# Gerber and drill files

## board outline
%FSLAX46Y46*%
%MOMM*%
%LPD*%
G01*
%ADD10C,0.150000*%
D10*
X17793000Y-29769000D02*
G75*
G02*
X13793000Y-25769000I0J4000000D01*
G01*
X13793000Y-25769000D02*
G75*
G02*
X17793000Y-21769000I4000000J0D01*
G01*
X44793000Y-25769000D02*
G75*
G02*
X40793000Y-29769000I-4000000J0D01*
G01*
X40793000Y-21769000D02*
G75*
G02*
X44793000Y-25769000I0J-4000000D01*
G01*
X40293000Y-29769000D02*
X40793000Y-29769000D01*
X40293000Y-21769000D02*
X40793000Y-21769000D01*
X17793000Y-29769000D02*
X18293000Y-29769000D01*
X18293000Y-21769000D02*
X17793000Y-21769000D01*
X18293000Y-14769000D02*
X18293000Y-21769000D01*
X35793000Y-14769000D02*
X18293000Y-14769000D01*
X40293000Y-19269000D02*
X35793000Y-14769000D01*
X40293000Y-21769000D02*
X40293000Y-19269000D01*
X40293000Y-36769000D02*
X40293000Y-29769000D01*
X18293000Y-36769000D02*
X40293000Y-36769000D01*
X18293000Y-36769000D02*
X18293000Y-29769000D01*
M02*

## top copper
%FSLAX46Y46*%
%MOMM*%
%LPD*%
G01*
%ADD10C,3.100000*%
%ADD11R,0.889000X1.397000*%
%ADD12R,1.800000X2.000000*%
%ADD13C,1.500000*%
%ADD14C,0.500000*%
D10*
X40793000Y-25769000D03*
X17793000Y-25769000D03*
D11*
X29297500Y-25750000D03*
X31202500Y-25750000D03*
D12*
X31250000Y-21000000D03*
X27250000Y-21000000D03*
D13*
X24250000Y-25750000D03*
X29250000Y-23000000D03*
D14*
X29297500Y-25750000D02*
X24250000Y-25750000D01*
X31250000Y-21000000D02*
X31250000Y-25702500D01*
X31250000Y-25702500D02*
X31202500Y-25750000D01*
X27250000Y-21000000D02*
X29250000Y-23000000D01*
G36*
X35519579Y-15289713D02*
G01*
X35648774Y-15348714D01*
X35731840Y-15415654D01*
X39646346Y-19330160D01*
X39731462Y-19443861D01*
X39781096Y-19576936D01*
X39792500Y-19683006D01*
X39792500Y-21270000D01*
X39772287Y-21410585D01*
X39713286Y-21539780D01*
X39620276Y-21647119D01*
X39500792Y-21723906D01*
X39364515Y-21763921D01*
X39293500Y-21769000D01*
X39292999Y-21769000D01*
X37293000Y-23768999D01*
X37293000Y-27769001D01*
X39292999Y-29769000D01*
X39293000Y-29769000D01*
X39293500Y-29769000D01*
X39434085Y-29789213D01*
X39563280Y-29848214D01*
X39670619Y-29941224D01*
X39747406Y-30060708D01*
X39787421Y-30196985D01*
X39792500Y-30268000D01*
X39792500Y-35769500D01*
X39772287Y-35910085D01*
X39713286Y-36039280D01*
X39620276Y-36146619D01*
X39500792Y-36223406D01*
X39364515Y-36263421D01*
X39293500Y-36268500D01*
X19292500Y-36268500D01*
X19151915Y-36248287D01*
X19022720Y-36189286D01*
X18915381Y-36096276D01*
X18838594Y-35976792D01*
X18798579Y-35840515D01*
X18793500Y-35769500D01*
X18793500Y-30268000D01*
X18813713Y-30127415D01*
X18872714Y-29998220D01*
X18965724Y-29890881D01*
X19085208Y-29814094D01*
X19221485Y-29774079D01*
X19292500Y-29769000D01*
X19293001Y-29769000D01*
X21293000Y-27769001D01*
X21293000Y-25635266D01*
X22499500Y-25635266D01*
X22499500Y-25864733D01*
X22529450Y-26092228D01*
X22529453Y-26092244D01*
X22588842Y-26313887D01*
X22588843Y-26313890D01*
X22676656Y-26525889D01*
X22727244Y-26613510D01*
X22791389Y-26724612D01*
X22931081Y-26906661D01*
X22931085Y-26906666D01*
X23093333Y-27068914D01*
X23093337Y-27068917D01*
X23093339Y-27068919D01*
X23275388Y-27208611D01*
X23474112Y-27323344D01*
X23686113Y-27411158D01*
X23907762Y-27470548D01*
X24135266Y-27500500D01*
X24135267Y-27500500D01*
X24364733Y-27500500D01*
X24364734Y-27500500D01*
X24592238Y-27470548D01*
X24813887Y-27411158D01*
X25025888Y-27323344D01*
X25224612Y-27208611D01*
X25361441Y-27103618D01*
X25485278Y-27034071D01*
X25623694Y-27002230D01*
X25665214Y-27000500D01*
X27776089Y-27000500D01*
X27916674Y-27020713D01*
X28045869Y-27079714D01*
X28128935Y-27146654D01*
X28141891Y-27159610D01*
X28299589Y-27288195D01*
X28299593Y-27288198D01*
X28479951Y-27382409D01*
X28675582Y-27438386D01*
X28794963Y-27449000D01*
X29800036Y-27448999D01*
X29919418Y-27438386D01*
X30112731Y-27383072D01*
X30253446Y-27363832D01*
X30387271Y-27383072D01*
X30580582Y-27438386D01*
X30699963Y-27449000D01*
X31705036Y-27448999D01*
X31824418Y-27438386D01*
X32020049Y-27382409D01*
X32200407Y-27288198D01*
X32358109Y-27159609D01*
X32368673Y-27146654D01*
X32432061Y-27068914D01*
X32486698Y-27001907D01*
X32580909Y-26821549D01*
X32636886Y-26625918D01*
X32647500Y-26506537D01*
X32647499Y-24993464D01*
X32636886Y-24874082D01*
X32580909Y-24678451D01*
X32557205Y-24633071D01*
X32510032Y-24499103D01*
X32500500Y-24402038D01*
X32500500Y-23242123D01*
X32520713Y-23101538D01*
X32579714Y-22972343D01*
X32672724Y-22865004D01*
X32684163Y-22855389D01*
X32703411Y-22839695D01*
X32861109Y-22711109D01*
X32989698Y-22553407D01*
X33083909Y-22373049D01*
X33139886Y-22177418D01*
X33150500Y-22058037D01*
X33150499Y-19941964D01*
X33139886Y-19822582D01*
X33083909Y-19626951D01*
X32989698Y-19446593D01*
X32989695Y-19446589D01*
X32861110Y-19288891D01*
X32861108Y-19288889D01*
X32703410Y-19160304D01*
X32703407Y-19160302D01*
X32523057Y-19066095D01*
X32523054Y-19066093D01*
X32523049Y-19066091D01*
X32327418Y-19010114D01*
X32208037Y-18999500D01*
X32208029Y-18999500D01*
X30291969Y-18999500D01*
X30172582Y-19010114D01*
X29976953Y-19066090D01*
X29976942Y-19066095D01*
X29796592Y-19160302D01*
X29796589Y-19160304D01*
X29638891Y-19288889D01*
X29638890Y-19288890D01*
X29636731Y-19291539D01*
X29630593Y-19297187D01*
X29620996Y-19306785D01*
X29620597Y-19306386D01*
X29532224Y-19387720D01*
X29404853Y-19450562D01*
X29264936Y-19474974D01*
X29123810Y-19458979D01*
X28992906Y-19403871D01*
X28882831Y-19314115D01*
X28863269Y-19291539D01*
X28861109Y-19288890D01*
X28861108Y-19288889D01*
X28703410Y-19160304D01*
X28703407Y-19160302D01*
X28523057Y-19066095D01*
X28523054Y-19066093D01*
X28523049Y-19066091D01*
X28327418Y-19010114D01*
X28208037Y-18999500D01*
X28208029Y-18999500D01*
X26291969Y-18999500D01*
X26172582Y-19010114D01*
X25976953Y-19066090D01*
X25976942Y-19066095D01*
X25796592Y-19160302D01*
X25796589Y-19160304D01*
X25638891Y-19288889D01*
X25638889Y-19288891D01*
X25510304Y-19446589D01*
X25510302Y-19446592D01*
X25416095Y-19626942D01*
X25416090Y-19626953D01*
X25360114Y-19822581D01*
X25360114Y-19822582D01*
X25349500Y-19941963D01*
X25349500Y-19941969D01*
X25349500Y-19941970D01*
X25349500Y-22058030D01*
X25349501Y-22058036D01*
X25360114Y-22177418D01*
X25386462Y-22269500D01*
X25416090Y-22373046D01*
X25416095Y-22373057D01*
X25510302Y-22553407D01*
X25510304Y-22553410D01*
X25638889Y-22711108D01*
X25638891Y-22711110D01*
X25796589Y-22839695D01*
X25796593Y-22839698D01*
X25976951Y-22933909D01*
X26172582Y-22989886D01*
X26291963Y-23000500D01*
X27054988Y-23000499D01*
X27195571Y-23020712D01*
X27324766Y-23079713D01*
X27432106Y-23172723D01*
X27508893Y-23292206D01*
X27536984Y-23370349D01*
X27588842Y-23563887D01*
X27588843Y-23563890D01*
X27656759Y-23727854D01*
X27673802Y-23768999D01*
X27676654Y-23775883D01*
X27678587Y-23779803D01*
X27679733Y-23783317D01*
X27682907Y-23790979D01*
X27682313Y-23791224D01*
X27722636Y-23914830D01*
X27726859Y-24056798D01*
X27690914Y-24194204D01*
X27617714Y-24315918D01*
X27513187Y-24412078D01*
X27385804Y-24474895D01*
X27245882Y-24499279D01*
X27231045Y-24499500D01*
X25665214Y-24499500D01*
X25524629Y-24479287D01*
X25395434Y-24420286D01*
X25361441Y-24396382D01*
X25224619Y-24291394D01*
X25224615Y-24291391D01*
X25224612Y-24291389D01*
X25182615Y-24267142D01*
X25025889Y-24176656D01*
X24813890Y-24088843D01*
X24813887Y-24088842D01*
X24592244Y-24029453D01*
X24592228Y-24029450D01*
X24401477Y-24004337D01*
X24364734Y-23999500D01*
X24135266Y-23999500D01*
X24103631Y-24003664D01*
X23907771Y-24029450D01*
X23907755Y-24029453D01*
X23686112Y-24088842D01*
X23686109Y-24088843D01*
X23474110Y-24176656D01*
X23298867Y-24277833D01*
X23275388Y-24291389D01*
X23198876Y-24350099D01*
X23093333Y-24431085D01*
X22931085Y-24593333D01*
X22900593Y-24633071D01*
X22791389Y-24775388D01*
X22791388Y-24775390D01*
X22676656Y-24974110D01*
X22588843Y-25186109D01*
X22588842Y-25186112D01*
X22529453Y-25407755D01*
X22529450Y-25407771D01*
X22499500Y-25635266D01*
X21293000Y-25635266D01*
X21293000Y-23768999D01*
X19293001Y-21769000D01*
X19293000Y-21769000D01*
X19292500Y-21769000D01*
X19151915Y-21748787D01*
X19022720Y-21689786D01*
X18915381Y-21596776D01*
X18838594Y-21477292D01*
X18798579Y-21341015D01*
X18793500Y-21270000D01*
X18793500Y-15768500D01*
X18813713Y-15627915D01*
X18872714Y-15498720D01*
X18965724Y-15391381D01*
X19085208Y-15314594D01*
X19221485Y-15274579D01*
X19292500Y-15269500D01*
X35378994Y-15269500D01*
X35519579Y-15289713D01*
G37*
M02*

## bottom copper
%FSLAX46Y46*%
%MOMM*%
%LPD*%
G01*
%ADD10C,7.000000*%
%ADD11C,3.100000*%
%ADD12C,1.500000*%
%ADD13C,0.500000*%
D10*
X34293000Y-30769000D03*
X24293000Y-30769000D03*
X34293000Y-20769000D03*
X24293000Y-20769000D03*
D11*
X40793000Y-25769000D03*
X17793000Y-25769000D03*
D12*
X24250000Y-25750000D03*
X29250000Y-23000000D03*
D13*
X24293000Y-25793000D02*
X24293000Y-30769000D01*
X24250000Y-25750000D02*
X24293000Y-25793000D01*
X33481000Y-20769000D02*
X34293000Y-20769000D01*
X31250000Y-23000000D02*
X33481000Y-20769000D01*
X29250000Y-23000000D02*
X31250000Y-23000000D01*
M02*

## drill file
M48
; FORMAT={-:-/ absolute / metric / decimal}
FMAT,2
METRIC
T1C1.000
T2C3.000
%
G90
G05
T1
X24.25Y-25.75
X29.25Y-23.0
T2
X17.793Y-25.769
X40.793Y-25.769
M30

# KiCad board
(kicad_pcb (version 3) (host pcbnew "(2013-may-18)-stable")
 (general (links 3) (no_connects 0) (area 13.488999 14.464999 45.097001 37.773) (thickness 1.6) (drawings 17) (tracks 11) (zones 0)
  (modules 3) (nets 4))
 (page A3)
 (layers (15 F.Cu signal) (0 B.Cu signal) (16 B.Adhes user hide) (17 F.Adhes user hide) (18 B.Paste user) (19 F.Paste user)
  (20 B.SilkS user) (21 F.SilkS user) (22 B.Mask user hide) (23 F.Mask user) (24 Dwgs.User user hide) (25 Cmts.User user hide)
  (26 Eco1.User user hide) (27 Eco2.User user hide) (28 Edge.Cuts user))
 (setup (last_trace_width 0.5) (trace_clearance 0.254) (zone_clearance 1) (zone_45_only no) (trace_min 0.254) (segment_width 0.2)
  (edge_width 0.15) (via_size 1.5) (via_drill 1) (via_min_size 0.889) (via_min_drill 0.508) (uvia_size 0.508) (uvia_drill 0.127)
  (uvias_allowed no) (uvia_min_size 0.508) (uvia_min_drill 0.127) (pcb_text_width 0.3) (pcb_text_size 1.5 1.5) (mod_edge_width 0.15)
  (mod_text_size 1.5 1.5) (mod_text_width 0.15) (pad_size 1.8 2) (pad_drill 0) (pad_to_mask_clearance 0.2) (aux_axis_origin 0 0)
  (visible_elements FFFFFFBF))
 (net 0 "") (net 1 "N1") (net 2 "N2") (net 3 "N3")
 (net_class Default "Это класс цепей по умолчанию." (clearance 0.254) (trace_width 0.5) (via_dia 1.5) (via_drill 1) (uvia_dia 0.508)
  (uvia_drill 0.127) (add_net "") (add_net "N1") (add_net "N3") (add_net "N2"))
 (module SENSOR (layer B.Cu) (at 40.793 37.269 180)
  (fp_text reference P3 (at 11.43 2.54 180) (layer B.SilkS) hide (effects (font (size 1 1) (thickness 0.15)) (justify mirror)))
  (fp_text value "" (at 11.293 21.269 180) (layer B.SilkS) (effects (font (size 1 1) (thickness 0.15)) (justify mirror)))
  (pad 2 smd circle (at 6.5 6.5 180) (size 7 7) (layers B.Cu B.Mask) (solder_mask_margin 0.1))
  (pad 3 smd circle (at 16.5 6.5 180) (size 7 7) (layers B.Cu B.Mask) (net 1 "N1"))
  (pad 1 smd circle (at 6.5 16.5 180) (size 7 7) (layers B.Cu B.Mask) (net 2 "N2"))
  (pad 4 smd circle (at 16.5 16.5 180) (size 7 7) (layers B.Cu B.Mask))
  (pad "" np_thru_hole circle (at 0 11.5 180) (size 3.1 3.1) (drill 3) (layers *.Cu *.Mask B.SilkS))
  (pad "" np_thru_hole circle (at 23 11.5 180) (size 3.1 3.1) (drill 3) (layers *.Cu *.Mask B.SilkS)))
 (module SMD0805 (layer F.Cu) (at 30.25 25.75)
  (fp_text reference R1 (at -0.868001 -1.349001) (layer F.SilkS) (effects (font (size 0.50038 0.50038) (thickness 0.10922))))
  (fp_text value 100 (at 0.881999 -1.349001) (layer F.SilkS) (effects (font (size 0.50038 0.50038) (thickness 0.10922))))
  (pad 1 smd rect (at -0.9525 0) (size 0.889 1.397) (layers F.Cu F.Paste F.Mask) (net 1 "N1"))
  (pad 2 smd rect (at 0.9525 0) (size 0.889 1.397) (layers F.Cu F.Paste F.Mask) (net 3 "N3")))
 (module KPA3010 (layer F.Cu) (at 29.25 21)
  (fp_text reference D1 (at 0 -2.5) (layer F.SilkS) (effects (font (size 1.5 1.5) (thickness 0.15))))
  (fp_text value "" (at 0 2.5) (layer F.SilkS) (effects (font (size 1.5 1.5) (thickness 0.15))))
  (pad 1 smd rect (at 2 0) (size 1.8 2) (layers F.Cu F.Paste F.Mask) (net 3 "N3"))
  (pad 2 smd rect (at -2 0) (size 1.8 2) (layers F.Cu F.Paste F.Mask) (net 2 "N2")))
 (gr_arc (start 17.793 25.769) (end 17.793 29.769) (angle 90) (layer Edge.Cuts) (width 0.15))
 (gr_arc (start 17.793 25.769) (end 13.793 25.769) (angle 90) (layer Edge.Cuts) (width 0.15))
 (gr_arc (start 40.793 25.769) (end 44.793 25.769) (angle 90) (layer Edge.Cuts) (width 0.15))
 (gr_arc (start 40.793 25.769) (end 40.793 21.769) (angle 90) (layer Edge.Cuts) (width 0.15))
 (gr_line (start 40.293 29.769) (end 40.793 29.769) (angle 90) (layer Edge.Cuts) (width 0.15))
 (gr_line (start 40.293 21.769) (end 40.793 21.769) (angle 90) (layer Edge.Cuts) (width 0.15))
 (gr_line (start 17.793 29.769) (end 18.293 29.769) (angle 90) (layer Edge.Cuts) (width 0.15))
 (gr_line (start 18.293 21.769) (end 17.793 21.769) (angle 90) (layer Edge.Cuts) (width 0.15))
 (gr_line (start 18.293 14.769) (end 18.293 21.769) (angle 90) (layer Edge.Cuts) (width 0.15))
 (gr_line (start 35.793 14.769) (end 18.293 14.769) (angle 90) (layer Edge.Cuts) (width 0.15))
 (gr_line (start 40.293 19.269) (end 35.793 14.769) (angle 90) (layer Edge.Cuts) (width 0.15))
 (gr_line (start 40.293 21.769) (end 40.293 19.269) (angle 90) (layer Edge.Cuts) (width 0.15))
 (gr_line (start 40.293 36.769) (end 40.293 29.769) (angle 90) (layer Edge.Cuts) (width 0.15))
 (gr_line (start 18.293 36.769) (end 40.293 36.769) (angle 90) (layer Edge.Cuts) (width 0.15))
 (gr_line (start 18.293 36.769) (end 18.293 29.769) (angle 90) (layer Edge.Cuts) (width 0.15))
 (segment (start 29.2975 25.75) (end 24.25 25.75) (width 0.5) (layer F.Cu) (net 1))
 (segment (start 24.293 25.793) (end 24.293 30.769) (width 0.5) (layer B.Cu) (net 1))
 (segment (start 24.25 25.75) (end 24.293 25.793) (width 0.5) (layer B.Cu) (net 1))
 (via (at 24.25 25.75) (size 1.5) (layers F.Cu B.Cu) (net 1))
 (segment (start 31.25 21) (end 31.25 25.7025) (width 0.5) (layer F.Cu) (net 3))
 (segment (start 31.25 25.7025) (end 31.2025 25.75) (width 0.5) (layer F.Cu) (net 3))
 (segment (start 27.25 21) (end 29.25 23) (width 0.5) (layer F.Cu) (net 2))
 (segment (start 33.481 20.769) (end 34.293 20.769) (width 0.5) (layer B.Cu) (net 2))
 (segment (start 31.25 23) (end 33.481 20.769) (width 0.5) (layer B.Cu) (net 2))
 (segment (start 29.25 23) (end 31.25 23) (width 0.5) (layer B.Cu) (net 2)) (via (at 29.25 23) (size 1.5) (layers F.Cu B.Cu) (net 2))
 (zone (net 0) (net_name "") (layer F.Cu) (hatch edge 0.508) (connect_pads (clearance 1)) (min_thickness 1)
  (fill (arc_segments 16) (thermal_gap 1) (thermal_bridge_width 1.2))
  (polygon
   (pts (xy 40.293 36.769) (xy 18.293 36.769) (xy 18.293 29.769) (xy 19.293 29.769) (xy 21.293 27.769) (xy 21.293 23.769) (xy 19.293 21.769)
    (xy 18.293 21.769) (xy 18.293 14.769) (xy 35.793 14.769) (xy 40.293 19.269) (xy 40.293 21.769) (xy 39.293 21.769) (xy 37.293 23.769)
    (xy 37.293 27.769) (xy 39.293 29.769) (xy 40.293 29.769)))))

